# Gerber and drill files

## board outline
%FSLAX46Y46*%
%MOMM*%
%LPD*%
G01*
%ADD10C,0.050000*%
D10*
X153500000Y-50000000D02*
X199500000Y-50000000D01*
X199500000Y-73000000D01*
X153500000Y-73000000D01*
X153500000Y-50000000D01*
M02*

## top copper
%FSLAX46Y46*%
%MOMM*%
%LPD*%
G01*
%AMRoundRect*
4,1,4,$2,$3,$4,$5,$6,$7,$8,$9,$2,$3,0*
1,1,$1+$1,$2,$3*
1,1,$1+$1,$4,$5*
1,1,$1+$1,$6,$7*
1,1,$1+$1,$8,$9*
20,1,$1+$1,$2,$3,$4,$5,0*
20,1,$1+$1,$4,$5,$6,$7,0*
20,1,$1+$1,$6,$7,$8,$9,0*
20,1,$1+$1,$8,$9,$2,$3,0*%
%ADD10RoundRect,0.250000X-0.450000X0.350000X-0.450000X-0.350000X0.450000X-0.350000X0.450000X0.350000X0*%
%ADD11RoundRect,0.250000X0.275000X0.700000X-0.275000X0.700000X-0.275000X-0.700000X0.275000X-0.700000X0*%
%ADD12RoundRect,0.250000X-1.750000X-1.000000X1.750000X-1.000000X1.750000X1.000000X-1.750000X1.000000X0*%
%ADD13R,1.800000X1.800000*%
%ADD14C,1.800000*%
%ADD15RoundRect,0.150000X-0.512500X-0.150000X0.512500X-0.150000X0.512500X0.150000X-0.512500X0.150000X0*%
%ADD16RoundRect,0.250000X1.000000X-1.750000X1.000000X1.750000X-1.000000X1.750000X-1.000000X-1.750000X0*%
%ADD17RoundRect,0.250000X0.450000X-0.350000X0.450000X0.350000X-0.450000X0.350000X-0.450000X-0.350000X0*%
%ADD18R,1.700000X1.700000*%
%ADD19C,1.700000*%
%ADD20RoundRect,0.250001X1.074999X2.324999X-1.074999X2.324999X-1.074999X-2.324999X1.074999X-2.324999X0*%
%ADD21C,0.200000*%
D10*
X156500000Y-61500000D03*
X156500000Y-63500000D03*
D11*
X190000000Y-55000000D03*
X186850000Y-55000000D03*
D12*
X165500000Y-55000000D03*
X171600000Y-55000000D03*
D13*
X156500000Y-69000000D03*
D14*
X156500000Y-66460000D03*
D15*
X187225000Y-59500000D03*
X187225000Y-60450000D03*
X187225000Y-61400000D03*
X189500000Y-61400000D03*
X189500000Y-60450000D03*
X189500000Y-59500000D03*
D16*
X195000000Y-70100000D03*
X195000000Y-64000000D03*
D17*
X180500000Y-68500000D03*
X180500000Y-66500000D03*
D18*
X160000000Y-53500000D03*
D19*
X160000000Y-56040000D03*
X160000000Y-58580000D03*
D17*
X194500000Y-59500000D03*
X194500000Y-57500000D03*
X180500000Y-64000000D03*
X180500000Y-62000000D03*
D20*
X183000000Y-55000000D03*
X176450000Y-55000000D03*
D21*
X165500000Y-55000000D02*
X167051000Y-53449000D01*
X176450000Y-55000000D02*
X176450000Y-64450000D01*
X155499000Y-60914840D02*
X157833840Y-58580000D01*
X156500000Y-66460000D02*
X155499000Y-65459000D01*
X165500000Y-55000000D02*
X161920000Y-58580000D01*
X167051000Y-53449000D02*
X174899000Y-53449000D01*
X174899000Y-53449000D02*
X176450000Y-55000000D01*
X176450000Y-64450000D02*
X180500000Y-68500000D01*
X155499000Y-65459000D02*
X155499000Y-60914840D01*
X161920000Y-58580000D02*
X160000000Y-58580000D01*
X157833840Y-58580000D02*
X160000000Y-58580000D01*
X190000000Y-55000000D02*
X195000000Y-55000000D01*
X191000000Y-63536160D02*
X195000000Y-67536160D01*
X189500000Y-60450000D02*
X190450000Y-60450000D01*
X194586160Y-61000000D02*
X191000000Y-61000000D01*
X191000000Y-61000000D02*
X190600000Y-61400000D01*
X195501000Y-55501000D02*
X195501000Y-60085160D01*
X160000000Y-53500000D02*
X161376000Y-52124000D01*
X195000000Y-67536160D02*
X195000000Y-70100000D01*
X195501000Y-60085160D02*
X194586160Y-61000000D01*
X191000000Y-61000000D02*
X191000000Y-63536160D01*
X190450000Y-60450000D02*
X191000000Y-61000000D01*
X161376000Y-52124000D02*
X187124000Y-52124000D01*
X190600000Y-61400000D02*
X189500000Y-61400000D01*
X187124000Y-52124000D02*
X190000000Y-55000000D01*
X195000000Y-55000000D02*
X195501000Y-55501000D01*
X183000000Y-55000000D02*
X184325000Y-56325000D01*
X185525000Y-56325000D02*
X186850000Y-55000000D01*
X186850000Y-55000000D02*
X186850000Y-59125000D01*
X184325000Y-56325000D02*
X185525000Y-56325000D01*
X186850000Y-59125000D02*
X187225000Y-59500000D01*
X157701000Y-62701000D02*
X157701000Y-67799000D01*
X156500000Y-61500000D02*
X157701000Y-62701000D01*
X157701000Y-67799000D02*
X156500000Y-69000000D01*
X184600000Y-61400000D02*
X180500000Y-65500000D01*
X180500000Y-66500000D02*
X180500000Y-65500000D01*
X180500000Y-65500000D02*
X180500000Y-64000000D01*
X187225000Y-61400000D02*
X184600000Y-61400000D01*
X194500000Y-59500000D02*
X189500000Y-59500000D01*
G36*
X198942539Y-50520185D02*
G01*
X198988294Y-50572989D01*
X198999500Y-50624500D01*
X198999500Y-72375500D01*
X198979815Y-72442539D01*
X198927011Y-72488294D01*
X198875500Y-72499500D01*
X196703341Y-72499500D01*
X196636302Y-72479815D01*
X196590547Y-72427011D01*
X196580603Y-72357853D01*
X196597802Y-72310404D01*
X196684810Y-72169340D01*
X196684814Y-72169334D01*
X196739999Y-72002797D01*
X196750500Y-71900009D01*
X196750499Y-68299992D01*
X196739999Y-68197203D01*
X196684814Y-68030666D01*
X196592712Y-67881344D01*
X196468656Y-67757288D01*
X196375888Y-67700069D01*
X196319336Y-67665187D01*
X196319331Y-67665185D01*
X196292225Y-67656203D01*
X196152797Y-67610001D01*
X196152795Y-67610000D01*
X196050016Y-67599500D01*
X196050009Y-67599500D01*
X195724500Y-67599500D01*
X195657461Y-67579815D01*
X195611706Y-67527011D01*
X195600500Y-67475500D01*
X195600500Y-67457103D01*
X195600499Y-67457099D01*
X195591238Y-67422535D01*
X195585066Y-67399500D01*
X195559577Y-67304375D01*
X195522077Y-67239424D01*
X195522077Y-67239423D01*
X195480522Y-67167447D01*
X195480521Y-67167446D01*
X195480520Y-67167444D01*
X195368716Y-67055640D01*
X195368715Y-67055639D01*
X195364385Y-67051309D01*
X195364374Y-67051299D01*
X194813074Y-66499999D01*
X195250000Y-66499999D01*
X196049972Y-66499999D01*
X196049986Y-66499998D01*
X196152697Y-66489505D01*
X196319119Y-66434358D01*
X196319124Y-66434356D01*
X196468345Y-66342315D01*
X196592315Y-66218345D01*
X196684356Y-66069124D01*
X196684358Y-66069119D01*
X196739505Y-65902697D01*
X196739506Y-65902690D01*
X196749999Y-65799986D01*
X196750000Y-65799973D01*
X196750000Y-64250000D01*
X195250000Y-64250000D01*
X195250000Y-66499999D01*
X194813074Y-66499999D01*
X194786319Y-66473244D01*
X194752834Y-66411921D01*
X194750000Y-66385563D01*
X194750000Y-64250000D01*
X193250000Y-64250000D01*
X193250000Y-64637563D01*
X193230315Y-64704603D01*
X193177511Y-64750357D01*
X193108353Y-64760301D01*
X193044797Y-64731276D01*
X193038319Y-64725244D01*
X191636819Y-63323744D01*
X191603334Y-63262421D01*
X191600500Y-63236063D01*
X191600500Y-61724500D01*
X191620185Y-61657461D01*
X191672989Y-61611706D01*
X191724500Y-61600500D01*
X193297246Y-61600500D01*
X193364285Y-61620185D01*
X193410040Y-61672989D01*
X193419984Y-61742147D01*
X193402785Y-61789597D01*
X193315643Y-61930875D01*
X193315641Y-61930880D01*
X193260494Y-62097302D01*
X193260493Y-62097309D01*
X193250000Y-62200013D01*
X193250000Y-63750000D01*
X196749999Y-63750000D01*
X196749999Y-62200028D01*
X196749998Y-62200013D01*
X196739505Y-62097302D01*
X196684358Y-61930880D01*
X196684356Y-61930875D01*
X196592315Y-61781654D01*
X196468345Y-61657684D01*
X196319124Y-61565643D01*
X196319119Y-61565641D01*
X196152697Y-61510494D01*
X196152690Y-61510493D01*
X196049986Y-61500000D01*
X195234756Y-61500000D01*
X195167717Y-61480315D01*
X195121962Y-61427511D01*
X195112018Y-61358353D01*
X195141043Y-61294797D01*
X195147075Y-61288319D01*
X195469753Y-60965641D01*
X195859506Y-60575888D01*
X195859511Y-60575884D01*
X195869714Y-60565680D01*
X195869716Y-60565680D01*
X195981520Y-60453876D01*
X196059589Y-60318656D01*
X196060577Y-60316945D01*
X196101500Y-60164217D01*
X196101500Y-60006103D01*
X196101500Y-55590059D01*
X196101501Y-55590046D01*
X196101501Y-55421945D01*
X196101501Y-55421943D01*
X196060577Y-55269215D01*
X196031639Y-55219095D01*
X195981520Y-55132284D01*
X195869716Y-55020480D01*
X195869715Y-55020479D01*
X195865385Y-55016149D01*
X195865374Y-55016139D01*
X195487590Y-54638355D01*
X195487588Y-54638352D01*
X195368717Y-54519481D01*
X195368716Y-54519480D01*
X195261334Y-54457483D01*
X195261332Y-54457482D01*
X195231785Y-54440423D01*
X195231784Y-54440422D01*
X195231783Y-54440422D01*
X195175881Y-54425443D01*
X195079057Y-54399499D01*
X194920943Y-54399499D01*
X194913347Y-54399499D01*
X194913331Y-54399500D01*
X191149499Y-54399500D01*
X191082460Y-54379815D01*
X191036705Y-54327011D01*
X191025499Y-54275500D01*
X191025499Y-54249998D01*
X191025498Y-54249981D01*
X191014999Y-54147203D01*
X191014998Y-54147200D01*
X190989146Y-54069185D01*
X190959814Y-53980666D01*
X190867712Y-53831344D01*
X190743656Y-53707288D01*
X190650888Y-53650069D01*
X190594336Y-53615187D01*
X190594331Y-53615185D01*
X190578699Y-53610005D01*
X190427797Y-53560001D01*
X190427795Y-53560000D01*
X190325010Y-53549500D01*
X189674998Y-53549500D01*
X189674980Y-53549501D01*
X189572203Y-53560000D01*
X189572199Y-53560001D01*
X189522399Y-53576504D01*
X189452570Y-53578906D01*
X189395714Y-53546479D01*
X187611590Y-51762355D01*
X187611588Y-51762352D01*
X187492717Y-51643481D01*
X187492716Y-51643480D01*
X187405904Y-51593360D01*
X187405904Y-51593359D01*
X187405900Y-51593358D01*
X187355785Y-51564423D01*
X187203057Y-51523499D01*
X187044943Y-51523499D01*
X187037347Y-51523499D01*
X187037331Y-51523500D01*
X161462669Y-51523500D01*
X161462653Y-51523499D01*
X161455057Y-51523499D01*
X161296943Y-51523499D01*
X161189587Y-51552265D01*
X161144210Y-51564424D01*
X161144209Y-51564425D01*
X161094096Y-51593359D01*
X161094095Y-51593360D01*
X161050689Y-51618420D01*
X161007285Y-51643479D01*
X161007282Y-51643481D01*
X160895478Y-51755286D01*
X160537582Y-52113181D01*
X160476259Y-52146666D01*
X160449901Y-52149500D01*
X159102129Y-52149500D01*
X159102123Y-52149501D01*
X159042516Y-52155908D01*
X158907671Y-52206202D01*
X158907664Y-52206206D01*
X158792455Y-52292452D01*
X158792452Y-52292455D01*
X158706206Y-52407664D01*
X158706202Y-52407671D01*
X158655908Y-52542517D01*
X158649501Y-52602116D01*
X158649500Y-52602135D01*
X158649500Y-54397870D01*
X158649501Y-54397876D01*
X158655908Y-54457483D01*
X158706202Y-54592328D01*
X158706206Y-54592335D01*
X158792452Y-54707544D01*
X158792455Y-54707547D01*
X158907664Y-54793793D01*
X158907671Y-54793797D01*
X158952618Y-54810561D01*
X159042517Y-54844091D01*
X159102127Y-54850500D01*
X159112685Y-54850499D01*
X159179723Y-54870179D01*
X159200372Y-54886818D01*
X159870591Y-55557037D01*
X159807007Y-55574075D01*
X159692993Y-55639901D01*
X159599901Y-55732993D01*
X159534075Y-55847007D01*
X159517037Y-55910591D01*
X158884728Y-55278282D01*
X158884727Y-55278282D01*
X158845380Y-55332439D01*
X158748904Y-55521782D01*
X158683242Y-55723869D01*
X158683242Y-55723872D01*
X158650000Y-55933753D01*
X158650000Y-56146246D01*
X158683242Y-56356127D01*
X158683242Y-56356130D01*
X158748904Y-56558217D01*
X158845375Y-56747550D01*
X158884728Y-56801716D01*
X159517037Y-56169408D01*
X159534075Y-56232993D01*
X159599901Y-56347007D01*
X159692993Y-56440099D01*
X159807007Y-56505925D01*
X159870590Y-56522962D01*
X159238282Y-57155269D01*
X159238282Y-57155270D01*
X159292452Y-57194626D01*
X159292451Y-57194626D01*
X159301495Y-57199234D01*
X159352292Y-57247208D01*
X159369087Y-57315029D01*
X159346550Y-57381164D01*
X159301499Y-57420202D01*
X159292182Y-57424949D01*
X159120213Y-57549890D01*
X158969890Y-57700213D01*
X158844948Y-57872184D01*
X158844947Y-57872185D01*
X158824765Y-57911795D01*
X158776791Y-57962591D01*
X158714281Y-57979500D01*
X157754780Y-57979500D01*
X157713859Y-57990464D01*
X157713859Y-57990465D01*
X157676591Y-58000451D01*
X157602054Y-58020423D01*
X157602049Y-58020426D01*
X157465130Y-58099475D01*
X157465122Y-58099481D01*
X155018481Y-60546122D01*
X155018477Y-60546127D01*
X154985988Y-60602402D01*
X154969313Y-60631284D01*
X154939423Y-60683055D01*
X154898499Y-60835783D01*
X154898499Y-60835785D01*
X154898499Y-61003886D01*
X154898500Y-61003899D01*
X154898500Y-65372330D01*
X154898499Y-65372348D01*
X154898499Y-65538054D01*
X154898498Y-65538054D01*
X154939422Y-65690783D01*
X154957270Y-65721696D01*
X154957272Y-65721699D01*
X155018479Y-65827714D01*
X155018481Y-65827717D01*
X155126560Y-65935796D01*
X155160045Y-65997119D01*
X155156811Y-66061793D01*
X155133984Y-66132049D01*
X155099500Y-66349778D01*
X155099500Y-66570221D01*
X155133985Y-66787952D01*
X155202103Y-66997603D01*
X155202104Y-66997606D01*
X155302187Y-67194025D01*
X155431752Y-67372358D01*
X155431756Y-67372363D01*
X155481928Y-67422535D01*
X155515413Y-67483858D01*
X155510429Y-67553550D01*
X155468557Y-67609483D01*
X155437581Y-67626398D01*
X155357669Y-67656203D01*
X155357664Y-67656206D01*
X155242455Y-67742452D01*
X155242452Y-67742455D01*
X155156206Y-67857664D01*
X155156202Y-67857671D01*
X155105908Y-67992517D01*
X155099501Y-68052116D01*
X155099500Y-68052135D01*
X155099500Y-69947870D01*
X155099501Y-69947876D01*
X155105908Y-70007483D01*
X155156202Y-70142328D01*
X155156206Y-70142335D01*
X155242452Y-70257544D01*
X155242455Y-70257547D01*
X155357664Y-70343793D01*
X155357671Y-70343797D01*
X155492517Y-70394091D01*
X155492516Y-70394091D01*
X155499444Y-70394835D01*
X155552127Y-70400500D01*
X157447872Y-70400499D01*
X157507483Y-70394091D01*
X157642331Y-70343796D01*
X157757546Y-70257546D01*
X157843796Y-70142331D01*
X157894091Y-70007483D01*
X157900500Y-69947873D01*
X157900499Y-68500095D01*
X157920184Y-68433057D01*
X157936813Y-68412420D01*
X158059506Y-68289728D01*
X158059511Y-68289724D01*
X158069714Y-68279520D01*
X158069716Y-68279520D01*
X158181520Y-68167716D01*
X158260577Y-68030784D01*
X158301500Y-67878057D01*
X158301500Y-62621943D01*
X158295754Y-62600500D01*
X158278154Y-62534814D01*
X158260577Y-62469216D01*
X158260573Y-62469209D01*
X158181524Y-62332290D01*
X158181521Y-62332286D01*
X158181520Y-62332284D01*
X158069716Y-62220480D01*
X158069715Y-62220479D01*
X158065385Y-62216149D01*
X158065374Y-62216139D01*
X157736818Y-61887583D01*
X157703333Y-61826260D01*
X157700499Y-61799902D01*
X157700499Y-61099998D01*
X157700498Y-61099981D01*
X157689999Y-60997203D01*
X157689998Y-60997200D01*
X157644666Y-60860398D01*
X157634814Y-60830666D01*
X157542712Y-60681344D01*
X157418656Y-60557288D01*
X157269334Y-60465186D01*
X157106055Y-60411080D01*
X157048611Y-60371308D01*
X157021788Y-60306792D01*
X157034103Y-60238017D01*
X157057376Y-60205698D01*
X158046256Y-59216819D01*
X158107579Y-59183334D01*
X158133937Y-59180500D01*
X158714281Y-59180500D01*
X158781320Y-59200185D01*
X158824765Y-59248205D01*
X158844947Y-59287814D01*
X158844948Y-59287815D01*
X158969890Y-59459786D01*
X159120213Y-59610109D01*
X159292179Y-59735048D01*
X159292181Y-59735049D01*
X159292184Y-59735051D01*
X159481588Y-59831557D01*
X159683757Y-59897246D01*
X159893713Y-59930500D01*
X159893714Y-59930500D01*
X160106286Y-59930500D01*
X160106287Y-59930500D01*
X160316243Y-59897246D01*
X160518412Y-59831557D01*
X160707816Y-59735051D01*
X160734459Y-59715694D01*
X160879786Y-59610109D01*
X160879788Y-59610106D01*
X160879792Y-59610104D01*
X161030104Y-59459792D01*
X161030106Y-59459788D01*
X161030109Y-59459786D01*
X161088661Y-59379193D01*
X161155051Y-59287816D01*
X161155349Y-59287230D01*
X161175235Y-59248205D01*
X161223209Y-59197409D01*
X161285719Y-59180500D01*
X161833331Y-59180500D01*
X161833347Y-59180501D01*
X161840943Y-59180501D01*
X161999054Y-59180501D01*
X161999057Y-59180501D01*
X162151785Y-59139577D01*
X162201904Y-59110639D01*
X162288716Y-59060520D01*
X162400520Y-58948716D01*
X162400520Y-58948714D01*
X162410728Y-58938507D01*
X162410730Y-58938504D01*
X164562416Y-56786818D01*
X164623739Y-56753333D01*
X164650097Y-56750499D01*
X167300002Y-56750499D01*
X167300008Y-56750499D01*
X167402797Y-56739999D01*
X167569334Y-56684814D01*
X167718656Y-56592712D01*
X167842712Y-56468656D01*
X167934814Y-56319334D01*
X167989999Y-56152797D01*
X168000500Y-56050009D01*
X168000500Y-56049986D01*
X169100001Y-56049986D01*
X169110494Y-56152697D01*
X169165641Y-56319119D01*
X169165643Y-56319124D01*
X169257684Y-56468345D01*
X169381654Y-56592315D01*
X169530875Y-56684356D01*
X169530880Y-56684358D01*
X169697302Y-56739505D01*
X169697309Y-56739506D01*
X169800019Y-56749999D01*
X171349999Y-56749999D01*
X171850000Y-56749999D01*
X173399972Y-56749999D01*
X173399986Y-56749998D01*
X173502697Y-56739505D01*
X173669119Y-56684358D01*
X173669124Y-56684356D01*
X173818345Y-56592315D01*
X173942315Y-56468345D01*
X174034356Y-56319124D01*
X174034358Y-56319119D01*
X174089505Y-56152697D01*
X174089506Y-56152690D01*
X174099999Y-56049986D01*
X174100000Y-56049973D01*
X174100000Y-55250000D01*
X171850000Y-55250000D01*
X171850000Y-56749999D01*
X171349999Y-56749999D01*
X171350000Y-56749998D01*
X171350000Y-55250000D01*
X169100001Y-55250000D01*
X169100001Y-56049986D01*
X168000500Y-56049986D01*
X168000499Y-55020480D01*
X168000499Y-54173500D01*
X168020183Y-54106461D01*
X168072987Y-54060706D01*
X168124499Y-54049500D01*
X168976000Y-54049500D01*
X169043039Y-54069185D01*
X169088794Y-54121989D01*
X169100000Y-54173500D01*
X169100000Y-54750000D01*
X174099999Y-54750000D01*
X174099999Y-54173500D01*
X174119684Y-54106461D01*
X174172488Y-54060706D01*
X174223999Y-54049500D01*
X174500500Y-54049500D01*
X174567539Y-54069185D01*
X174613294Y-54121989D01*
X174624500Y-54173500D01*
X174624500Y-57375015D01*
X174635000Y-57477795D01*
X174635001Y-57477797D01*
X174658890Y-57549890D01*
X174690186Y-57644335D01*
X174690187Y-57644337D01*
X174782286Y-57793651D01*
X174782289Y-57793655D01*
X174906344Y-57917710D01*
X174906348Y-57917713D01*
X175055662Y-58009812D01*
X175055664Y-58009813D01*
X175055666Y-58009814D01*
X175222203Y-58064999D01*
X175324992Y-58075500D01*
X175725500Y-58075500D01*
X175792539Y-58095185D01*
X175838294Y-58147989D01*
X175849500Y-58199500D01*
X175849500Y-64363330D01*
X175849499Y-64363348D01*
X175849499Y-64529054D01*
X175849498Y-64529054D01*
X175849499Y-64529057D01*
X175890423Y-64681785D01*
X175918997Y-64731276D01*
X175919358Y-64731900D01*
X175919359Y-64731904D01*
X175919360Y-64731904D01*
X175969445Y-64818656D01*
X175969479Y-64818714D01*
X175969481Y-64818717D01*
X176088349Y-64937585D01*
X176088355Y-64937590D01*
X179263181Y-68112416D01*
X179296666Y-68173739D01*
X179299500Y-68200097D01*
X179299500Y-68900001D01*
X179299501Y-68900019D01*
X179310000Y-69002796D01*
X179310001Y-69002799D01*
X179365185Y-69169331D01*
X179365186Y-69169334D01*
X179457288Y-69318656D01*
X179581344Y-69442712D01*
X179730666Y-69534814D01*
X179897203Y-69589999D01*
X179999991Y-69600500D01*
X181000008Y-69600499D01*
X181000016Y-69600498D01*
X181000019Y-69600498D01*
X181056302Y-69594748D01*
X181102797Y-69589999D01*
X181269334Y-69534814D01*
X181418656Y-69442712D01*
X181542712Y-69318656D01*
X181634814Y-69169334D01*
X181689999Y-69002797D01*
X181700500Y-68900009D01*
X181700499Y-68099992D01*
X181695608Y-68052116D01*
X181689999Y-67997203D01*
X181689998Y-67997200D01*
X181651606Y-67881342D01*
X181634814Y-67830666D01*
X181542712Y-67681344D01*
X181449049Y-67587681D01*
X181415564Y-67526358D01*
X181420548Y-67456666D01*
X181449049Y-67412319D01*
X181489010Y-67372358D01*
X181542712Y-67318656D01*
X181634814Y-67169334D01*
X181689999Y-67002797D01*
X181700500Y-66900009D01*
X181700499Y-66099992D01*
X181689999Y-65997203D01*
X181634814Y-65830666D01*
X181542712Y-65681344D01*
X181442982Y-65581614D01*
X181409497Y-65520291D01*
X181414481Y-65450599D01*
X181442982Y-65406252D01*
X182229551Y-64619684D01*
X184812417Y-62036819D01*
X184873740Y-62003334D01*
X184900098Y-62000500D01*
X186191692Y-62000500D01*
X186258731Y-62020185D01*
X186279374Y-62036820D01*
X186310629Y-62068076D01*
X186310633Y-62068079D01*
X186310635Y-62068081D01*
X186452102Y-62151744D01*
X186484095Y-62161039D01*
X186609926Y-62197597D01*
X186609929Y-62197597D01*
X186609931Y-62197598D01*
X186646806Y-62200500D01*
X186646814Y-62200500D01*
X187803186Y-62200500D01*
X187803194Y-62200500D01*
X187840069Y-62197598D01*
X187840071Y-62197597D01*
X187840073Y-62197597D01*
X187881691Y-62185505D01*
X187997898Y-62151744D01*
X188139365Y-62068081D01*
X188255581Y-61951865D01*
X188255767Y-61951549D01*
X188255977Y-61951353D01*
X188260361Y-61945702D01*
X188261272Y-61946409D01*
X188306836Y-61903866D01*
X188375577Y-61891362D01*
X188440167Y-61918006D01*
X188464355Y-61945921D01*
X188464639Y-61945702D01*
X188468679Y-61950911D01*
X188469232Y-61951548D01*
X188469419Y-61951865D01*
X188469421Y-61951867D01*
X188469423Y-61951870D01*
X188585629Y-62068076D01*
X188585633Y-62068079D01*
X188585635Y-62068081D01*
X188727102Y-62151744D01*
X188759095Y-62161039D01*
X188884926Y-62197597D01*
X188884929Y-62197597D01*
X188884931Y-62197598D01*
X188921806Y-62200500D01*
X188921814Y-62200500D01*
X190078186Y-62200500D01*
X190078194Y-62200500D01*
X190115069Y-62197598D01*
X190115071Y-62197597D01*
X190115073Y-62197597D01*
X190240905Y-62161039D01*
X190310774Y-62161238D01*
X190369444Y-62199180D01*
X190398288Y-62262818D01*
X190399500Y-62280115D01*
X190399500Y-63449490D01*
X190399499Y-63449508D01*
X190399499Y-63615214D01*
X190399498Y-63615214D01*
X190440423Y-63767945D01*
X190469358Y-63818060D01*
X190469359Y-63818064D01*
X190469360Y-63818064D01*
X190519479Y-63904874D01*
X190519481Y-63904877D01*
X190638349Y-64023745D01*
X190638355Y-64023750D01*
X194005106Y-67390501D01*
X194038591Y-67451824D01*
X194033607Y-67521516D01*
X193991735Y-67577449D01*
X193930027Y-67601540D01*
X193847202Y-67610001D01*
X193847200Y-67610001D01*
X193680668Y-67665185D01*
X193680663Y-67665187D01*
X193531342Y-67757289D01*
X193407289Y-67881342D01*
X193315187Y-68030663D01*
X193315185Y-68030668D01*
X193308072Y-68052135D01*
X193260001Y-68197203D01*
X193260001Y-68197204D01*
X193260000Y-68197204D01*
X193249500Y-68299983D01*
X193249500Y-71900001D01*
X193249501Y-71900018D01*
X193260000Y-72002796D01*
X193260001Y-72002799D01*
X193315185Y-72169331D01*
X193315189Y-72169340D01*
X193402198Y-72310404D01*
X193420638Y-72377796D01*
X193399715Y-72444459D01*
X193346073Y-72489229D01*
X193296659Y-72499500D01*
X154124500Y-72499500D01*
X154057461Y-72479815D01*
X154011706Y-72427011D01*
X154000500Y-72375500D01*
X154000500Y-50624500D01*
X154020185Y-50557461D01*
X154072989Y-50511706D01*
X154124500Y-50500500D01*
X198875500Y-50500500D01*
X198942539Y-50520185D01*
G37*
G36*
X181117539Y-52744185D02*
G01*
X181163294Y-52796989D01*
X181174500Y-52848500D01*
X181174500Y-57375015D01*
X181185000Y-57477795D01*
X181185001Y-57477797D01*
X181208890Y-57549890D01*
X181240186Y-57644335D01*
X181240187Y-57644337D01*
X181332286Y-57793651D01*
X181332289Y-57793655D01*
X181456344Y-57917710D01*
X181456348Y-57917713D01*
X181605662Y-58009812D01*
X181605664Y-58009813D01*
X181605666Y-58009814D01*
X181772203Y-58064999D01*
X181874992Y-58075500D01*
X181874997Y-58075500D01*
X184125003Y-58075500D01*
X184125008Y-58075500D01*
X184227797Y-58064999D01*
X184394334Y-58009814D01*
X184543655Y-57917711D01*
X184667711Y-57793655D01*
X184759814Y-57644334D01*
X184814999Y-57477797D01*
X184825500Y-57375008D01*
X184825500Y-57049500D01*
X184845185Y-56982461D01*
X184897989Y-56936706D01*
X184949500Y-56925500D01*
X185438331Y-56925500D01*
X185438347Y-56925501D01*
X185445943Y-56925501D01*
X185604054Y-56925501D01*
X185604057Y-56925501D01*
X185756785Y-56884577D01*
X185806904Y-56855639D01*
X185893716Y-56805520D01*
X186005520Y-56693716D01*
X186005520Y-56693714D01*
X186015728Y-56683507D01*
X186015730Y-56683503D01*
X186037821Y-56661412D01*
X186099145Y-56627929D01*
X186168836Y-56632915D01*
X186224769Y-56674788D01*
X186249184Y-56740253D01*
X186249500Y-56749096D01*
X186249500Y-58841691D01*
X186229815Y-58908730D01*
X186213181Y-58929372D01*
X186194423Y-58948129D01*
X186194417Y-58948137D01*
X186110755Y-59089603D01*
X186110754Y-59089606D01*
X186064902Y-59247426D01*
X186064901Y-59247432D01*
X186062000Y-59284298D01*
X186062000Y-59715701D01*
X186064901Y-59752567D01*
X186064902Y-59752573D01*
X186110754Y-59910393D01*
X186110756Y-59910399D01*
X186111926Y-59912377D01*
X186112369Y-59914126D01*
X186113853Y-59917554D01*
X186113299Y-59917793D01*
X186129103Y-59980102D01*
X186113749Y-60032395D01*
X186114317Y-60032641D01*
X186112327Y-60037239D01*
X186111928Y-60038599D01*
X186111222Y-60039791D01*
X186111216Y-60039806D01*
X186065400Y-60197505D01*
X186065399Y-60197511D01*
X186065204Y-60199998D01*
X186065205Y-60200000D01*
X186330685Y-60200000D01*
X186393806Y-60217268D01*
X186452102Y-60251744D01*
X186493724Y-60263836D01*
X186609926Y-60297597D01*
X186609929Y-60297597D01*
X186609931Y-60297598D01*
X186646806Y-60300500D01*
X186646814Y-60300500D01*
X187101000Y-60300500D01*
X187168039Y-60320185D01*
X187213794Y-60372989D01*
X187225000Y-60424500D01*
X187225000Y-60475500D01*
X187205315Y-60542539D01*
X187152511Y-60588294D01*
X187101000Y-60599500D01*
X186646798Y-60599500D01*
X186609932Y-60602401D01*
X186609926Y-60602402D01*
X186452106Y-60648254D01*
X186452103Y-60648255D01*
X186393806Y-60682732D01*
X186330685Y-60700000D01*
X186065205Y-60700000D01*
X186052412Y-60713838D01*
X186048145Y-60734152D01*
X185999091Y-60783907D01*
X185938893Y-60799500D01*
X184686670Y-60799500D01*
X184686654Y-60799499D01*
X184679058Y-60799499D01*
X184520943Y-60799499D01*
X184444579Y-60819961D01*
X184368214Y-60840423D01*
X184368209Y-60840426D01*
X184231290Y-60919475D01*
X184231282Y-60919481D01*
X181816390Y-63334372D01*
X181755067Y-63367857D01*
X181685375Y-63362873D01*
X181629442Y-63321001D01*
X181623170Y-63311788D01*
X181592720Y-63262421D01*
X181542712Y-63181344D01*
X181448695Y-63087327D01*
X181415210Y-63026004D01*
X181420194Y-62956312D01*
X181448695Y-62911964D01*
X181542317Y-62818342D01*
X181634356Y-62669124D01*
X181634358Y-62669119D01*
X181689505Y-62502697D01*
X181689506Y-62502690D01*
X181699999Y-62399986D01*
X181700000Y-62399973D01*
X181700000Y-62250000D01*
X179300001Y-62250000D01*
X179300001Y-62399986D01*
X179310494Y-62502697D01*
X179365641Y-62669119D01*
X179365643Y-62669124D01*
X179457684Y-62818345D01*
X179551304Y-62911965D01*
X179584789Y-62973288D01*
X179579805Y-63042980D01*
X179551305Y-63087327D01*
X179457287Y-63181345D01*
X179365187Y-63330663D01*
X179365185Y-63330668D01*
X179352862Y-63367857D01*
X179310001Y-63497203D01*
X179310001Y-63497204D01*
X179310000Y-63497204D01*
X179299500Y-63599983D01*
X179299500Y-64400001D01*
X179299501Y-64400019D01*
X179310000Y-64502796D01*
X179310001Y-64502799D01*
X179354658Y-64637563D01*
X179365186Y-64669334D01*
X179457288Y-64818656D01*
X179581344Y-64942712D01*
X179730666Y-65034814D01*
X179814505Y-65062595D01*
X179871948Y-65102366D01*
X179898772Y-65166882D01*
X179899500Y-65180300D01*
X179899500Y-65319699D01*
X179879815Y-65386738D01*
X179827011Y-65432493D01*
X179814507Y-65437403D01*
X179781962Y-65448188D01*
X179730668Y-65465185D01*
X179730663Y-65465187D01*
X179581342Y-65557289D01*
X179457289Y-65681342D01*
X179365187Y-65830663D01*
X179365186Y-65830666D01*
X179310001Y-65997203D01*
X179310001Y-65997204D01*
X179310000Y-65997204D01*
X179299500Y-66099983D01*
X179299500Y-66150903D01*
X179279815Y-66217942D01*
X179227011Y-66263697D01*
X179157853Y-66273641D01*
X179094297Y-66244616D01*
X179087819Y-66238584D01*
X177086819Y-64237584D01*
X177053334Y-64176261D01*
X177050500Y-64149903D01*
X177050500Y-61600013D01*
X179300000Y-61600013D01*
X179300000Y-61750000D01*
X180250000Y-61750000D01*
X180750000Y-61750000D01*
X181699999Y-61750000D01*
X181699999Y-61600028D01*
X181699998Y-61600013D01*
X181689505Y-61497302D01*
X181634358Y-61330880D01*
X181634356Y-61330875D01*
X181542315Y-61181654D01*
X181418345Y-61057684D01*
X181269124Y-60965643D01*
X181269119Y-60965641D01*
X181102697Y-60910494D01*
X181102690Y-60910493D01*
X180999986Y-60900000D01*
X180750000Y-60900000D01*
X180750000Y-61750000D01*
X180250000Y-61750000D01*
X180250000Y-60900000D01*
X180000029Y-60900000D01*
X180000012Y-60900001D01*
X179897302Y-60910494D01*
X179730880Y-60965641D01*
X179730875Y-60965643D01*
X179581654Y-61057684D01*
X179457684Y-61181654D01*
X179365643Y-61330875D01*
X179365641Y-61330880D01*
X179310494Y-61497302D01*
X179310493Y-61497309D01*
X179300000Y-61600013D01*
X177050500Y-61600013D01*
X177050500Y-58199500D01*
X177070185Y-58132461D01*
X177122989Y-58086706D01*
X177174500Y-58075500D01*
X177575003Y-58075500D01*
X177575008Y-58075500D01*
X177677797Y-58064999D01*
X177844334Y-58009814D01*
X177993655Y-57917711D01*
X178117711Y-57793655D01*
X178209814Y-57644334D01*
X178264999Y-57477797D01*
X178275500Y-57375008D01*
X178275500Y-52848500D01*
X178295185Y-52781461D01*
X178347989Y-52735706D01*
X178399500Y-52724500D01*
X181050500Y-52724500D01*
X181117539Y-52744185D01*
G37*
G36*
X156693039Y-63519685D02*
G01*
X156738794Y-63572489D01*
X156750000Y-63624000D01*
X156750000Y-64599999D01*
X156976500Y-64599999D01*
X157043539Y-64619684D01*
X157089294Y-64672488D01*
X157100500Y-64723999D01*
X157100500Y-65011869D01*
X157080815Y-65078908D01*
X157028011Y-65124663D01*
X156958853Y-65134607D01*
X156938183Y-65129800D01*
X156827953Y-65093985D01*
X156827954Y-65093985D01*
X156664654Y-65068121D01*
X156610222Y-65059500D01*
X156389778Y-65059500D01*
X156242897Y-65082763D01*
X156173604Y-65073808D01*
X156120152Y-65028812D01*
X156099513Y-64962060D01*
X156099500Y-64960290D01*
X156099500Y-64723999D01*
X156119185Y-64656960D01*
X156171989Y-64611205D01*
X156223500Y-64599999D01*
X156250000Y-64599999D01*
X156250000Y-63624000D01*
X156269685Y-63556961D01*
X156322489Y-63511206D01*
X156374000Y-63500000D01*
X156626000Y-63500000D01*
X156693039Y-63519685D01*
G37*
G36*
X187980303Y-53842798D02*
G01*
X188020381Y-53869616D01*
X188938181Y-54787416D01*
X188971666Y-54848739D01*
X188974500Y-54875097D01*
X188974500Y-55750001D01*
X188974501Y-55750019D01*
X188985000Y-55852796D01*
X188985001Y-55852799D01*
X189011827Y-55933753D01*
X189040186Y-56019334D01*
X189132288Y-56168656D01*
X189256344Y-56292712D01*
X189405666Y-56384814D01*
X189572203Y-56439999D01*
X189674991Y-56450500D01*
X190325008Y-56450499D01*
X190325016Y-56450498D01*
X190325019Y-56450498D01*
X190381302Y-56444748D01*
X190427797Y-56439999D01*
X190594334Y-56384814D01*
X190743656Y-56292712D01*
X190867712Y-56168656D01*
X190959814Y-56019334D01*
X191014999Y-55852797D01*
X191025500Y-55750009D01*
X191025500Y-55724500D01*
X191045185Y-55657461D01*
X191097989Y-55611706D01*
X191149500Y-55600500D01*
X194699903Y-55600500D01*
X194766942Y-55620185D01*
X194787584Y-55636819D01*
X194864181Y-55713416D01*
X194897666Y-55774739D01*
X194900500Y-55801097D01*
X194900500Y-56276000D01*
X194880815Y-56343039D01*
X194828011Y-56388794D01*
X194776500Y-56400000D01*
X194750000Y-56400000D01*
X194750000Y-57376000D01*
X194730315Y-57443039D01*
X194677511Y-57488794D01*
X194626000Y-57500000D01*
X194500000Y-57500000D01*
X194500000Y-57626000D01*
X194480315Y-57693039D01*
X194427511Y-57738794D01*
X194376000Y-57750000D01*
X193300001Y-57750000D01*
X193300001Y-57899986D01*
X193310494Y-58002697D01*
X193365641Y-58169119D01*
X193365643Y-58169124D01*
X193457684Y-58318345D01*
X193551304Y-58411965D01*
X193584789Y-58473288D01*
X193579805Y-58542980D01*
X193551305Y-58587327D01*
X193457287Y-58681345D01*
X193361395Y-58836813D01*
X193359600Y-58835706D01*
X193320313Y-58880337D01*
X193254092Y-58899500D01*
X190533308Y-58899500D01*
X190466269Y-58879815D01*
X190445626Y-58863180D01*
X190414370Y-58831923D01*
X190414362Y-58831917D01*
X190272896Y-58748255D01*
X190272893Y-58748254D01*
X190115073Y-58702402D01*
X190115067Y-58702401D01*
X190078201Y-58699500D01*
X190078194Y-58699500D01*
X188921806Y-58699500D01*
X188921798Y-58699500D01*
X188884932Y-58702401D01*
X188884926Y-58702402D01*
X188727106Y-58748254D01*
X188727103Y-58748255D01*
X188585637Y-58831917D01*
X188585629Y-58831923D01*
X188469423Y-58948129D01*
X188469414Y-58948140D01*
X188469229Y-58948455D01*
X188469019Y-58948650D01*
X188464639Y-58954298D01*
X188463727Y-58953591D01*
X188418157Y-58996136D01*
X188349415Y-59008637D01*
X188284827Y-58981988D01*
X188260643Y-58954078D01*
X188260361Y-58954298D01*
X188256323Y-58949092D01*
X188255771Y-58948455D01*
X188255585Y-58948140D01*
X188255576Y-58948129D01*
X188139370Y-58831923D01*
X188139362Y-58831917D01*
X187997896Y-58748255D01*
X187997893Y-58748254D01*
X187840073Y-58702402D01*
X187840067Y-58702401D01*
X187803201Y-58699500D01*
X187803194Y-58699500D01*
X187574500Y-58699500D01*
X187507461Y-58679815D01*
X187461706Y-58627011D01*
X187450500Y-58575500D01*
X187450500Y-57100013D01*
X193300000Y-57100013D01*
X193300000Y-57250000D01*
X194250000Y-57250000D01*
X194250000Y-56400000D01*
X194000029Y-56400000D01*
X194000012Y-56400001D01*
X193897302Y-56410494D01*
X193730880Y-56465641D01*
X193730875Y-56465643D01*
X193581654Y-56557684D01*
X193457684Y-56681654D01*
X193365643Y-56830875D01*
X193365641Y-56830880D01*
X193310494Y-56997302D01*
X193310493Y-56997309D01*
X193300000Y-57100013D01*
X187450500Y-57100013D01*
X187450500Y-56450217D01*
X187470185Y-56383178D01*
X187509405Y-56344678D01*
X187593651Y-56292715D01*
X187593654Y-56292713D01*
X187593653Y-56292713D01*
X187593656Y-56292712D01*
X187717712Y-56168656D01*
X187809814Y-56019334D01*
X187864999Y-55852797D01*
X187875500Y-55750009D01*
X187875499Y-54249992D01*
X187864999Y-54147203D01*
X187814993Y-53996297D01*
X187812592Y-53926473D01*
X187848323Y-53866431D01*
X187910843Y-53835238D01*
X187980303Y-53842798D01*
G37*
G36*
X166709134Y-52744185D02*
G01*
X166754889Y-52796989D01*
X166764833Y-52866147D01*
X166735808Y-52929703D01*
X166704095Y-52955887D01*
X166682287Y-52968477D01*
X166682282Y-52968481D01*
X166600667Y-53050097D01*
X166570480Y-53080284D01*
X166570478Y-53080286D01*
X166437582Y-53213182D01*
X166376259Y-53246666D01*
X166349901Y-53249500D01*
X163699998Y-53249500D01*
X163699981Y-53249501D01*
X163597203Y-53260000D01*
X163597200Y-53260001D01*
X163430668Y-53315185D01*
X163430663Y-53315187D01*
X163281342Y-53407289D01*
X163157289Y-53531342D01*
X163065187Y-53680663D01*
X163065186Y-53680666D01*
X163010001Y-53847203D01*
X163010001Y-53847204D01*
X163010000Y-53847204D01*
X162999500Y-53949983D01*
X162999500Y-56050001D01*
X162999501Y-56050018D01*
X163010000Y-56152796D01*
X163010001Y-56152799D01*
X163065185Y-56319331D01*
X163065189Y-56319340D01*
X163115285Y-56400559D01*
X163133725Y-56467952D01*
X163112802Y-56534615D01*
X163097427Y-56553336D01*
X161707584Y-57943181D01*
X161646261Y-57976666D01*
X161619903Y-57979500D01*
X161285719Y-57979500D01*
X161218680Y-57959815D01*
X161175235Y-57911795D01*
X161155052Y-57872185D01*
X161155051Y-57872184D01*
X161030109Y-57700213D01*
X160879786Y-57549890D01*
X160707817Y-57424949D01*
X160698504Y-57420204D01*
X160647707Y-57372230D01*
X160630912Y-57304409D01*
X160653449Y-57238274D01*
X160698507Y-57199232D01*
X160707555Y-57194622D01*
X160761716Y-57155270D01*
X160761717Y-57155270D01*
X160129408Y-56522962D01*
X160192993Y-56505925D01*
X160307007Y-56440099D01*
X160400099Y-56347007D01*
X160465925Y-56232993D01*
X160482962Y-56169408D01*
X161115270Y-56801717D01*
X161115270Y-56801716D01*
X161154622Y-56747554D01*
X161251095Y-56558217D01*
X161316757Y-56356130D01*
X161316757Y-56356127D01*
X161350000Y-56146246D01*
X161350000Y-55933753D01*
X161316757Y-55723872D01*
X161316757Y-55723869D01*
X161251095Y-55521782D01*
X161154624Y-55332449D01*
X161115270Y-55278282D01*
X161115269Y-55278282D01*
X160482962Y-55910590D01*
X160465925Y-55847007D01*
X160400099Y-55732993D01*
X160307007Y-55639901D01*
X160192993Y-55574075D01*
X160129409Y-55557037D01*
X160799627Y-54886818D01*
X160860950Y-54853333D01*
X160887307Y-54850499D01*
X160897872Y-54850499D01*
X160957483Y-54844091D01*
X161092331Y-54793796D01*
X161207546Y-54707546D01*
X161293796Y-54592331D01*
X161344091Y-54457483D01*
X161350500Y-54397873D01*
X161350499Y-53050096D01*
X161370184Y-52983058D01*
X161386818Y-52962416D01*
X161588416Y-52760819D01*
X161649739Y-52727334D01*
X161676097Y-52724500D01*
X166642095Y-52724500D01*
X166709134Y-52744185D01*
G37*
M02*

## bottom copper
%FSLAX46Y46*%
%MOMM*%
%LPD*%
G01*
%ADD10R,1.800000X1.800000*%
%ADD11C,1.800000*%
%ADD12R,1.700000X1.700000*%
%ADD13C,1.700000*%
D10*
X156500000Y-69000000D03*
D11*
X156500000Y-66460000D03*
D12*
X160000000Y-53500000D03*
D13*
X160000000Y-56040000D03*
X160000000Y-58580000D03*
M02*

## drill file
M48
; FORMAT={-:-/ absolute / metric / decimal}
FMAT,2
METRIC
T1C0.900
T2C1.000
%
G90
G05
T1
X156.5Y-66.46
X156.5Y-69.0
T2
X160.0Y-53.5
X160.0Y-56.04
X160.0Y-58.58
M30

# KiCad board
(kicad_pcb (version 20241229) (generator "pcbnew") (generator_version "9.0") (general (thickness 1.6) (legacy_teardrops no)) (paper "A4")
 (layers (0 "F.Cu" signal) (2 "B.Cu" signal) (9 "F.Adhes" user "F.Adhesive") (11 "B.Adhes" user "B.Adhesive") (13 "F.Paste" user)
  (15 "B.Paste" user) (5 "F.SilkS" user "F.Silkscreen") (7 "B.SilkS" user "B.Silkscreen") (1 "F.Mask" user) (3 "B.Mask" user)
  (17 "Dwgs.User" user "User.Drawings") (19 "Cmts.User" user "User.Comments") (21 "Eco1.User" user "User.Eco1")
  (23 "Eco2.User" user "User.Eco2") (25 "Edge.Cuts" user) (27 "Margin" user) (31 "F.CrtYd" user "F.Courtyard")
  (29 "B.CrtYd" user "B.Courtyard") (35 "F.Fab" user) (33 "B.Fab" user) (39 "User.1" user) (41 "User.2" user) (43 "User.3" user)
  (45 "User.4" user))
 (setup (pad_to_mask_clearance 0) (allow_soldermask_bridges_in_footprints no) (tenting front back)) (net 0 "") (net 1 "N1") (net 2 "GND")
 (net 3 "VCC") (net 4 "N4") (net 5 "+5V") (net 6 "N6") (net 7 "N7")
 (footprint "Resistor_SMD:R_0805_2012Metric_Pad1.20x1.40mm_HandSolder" (layer "F.Cu") (at 156.5 62.5 -90)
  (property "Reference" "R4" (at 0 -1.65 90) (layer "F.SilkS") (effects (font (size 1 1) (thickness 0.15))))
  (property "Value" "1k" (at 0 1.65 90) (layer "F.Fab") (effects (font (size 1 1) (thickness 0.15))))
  (pad "1" smd roundrect (at -1 0 270) (size 1.2 1.4) (layers "F.Cu" "F.Mask" "F.Paste") (roundrect_rratio 0.208333) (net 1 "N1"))
  (pad "2" smd roundrect (at 1 0 270) (size 1.2 1.4) (layers "F.Cu" "F.Mask" "F.Paste") (roundrect_rratio 0.208333) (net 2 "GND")))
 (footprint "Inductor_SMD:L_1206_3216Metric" (layer "F.Cu") (at 188.425 55 180)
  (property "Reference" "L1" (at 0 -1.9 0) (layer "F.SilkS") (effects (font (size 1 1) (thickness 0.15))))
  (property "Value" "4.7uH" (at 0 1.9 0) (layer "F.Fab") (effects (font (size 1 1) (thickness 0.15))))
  (pad "1" smd roundrect (at -1.575 0 180) (size 1.05 1.9) (layers "F.Cu" "F.Mask" "F.Paste") (roundrect_rratio 0.238095) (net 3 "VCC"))
  (pad "2" smd roundrect (at 1.575 0 180) (size 1.05 1.9) (layers "F.Cu" "F.Mask" "F.Paste") (roundrect_rratio 0.238095) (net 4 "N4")))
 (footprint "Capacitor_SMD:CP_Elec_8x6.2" (layer "F.Cu") (at 168.55 55)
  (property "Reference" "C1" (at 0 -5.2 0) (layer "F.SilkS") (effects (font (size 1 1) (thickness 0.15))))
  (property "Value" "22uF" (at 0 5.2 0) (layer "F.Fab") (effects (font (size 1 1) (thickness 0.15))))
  (pad "1" smd roundrect (at -3.05 0) (size 4 2.5) (layers "F.Cu" "F.Mask" "F.Paste") (roundrect_rratio 0.1) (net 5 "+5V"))
  (pad "2" smd roundrect (at 3.05 0) (size 4 2.5) (layers "F.Cu" "F.Mask" "F.Paste") (roundrect_rratio 0.1) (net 2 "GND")))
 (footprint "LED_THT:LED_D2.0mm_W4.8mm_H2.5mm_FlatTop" (layer "F.Cu") (at 156.5 69 90)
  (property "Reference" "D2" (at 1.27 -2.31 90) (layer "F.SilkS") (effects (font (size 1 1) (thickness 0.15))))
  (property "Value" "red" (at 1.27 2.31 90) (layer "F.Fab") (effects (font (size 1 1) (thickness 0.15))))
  (pad "1" thru_hole rect (at 0 0 90) (size 1.8 1.8) (drill 0.9) (layers "*.Cu" "*.Mask") (remove_unused_layers no) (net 1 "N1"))
  (pad "2" thru_hole circle (at 2.54 0 90) (size 1.8 1.8) (drill 0.9) (layers "*.Cu" "*.Mask") (remove_unused_layers no) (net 5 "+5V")))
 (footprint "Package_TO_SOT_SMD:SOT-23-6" (layer "F.Cu") (at 188.3625 60.45)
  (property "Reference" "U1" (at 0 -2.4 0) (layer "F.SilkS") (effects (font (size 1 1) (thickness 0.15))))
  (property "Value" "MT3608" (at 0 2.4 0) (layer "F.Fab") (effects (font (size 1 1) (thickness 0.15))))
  (pad "1" smd roundrect (at -1.1375 -0.95) (size 1.325 0.6) (layers "F.Cu" "F.Mask" "F.Paste") (roundrect_rratio 0.25) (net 4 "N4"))
  (pad "2" smd roundrect (at -1.1375 0) (size 1.325 0.6) (layers "F.Cu" "F.Mask" "F.Paste") (roundrect_rratio 0.25) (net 2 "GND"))
  (pad "3" smd roundrect (at -1.1375 0.95) (size 1.325 0.6) (layers "F.Cu" "F.Mask" "F.Paste") (roundrect_rratio 0.25) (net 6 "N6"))
  (pad "4" smd roundrect (at 1.1375 0.95) (size 1.325 0.6) (layers "F.Cu" "F.Mask" "F.Paste") (roundrect_rratio 0.25) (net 3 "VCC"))
  (pad "5" smd roundrect (at 1.1375 0) (size 1.325 0.6) (layers "F.Cu" "F.Mask" "F.Paste") (roundrect_rratio 0.25) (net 3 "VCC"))
  (pad "6" smd roundrect (at 1.1375 -0.95) (size 1.325 0.6) (layers "F.Cu" "F.Mask" "F.Paste") (roundrect_rratio 0.25) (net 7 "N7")))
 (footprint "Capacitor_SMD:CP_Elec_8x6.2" (layer "F.Cu") (at 195 67.05 90)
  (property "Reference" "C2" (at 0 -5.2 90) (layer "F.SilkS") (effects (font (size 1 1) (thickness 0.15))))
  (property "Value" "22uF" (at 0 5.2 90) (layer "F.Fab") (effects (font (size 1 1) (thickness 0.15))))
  (pad "1" smd roundrect (at -3.05 0 90) (size 4 2.5) (layers "F.Cu" "F.Mask" "F.Paste") (roundrect_rratio 0.1) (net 3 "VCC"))
  (pad "2" smd roundrect (at 3.05 0 90) (size 4 2.5) (layers "F.Cu" "F.Mask" "F.Paste") (roundrect_rratio 0.1) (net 2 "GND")))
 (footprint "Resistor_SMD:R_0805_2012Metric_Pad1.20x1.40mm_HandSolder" (layer "F.Cu") (at 180.5 67.5 90)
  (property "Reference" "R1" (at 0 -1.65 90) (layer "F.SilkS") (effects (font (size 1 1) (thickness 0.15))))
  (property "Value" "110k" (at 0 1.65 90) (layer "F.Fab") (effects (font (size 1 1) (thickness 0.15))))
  (pad "1" smd roundrect (at -1 0 90) (size 1.2 1.4) (layers "F.Cu" "F.Mask" "F.Paste") (roundrect_rratio 0.208333) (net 5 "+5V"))
  (pad "2" smd roundrect (at 1 0 90) (size 1.2 1.4) (layers "F.Cu" "F.Mask" "F.Paste") (roundrect_rratio 0.208333) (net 6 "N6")))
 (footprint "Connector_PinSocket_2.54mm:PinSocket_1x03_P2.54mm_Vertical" (layer "F.Cu") (at 160 53.5)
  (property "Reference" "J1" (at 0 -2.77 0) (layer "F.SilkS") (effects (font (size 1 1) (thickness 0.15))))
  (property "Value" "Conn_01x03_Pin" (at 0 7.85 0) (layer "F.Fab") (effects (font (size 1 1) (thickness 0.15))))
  (pad "1" thru_hole rect (at 0 0) (size 1.7 1.7) (drill 1) (layers "*.Cu" "*.Mask") (remove_unused_layers no) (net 3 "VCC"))
  (pad "2" thru_hole circle (at 0 2.54) (size 1.7 1.7) (drill 1) (layers "*.Cu" "*.Mask") (remove_unused_layers no) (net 2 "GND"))
  (pad "3" thru_hole circle (at 0 5.08) (size 1.7 1.7) (drill 1) (layers "*.Cu" "*.Mask") (remove_unused_layers no) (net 5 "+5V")))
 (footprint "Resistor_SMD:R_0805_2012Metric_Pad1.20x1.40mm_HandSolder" (layer "F.Cu") (at 194.5 58.5 90)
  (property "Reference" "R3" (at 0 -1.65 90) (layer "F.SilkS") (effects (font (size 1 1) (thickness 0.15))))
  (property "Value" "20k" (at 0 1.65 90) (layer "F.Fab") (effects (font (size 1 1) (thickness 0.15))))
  (pad "1" smd roundrect (at -1 0 90) (size 1.2 1.4) (layers "F.Cu" "F.Mask" "F.Paste") (roundrect_rratio 0.208333) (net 7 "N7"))
  (pad "2" smd roundrect (at 1 0 90) (size 1.2 1.4) (layers "F.Cu" "F.Mask" "F.Paste") (roundrect_rratio 0.208333) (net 2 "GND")))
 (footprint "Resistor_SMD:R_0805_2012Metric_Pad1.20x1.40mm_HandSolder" (layer "F.Cu") (at 180.5 63 90)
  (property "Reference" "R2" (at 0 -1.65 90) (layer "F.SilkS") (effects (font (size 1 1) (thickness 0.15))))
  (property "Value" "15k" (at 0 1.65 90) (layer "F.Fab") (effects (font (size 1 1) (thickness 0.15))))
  (pad "1" smd roundrect (at -1 0 90) (size 1.2 1.4) (layers "F.Cu" "F.Mask" "F.Paste") (roundrect_rratio 0.208333) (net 6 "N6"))
  (pad "2" smd roundrect (at 1 0 90) (size 1.2 1.4) (layers "F.Cu" "F.Mask" "F.Paste") (roundrect_rratio 0.208333) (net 2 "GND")))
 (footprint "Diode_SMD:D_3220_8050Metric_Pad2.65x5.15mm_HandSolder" (layer "F.Cu") (at 179.725 55 180)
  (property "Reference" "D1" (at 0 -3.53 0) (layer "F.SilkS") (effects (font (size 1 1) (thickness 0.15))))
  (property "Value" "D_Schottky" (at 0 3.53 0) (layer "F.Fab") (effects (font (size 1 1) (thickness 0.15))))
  (pad "1" smd roundrect (at -3.275 0 180) (size 2.65 5.15) (layers "F.Cu" "F.Mask" "F.Paste") (roundrect_rratio 0.09434) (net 4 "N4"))
  (pad "2" smd roundrect (at 3.275 0 180) (size 2.65 5.15) (layers "F.Cu" "F.Mask" "F.Paste") (roundrect_rratio 0.09434) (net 5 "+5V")))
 (gr_rect (start 153.5 50) (end 199.5 73) (stroke (width 0.05) (type default)) (fill no) (layer "Edge.Cuts"))
 (segment (start 165.5 55) (end 167.051 53.449) (width 0.2) (layer "F.Cu") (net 5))
 (segment (start 176.45 55) (end 176.45 64.45) (width 0.2) (layer "F.Cu") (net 5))
 (segment (start 155.499 60.91484) (end 157.83384 58.58) (width 0.2) (layer "F.Cu") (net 5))
 (segment (start 156.5 66.46) (end 155.499 65.459) (width 0.2) (layer "F.Cu") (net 5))
 (segment (start 165.5 55) (end 161.92 58.58) (width 0.2) (layer "F.Cu") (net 5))
 (segment (start 167.051 53.449) (end 174.899 53.449) (width 0.2) (layer "F.Cu") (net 5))
 (segment (start 174.899 53.449) (end 176.45 55) (width 0.2) (layer "F.Cu") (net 5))
 (segment (start 176.45 64.45) (end 180.5 68.5) (width 0.2) (layer "F.Cu") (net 5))
 (segment (start 155.499 65.459) (end 155.499 60.91484) (width 0.2) (layer "F.Cu") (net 5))
 (segment (start 161.92 58.58) (end 160 58.58) (width 0.2) (layer "F.Cu") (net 5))
 (segment (start 157.83384 58.58) (end 160 58.58) (width 0.2) (layer "F.Cu") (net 5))
 (segment (start 190 55) (end 195 55) (width 0.2) (layer "F.Cu") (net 3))
 (segment (start 191 63.53616) (end 195 67.53616) (width 0.2) (layer "F.Cu") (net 3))
 (segment (start 189.5 60.45) (end 190.45 60.45) (width 0.2) (layer "F.Cu") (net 3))
 (segment (start 194.58616 61) (end 191 61) (width 0.2) (layer "F.Cu") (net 3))
 (segment (start 191 61) (end 190.6 61.4) (width 0.2) (layer "F.Cu") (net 3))
 (segment (start 195.501 55.501) (end 195.501 60.08516) (width 0.2) (layer "F.Cu") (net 3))
 (segment (start 160 53.5) (end 161.376 52.124) (width 0.2) (layer "F.Cu") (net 3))
 (segment (start 195 67.53616) (end 195 70.1) (width 0.2) (layer "F.Cu") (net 3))
 (segment (start 195.501 60.08516) (end 194.58616 61) (width 0.2) (layer "F.Cu") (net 3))
 (segment (start 191 61) (end 191 63.53616) (width 0.2) (layer "F.Cu") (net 3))
 (segment (start 190.45 60.45) (end 191 61) (width 0.2) (layer "F.Cu") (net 3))
 (segment (start 161.376 52.124) (end 187.124 52.124) (width 0.2) (layer "F.Cu") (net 3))
 (segment (start 190.6 61.4) (end 189.5 61.4) (width 0.2) (layer "F.Cu") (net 3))
 (segment (start 187.124 52.124) (end 190 55) (width 0.2) (layer "F.Cu") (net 3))
 (segment (start 195 55) (end 195.501 55.501) (width 0.2) (layer "F.Cu") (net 3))
 (segment (start 183 55) (end 184.325 56.325) (width 0.2) (layer "F.Cu") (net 4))
 (segment (start 185.525 56.325) (end 186.85 55) (width 0.2) (layer "F.Cu") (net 4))
 (segment (start 186.85 55) (end 186.85 59.125) (width 0.2) (layer "F.Cu") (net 4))
 (segment (start 184.325 56.325) (end 185.525 56.325) (width 0.2) (layer "F.Cu") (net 4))
 (segment (start 186.85 59.125) (end 187.225 59.5) (width 0.2) (layer "F.Cu") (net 4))
 (segment (start 157.701 62.701) (end 157.701 67.799) (width 0.2) (layer "F.Cu") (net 1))
 (segment (start 156.5 61.5) (end 157.701 62.701) (width 0.2) (layer "F.Cu") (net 1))
 (segment (start 157.701 67.799) (end 156.5 69) (width 0.2) (layer "F.Cu") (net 1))
 (segment (start 184.6 61.4) (end 180.5 65.5) (width 0.2) (layer "F.Cu") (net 6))
 (segment (start 180.5 66.5) (end 180.5 65.5) (width 0.2) (layer "F.Cu") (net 6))
 (segment (start 180.5 65.5) (end 180.5 64) (width 0.2) (layer "F.Cu") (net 6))
 (segment (start 187.225 61.4) (end 184.6 61.4) (width 0.2) (layer "F.Cu") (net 6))
 (segment (start 194.5 59.5) (end 189.5 59.5) (width 0.2) (layer "F.Cu") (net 7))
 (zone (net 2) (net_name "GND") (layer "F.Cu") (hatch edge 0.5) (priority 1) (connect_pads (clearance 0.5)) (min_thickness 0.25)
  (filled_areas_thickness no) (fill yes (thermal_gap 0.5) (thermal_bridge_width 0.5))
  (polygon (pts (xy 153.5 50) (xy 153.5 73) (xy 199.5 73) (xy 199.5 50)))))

